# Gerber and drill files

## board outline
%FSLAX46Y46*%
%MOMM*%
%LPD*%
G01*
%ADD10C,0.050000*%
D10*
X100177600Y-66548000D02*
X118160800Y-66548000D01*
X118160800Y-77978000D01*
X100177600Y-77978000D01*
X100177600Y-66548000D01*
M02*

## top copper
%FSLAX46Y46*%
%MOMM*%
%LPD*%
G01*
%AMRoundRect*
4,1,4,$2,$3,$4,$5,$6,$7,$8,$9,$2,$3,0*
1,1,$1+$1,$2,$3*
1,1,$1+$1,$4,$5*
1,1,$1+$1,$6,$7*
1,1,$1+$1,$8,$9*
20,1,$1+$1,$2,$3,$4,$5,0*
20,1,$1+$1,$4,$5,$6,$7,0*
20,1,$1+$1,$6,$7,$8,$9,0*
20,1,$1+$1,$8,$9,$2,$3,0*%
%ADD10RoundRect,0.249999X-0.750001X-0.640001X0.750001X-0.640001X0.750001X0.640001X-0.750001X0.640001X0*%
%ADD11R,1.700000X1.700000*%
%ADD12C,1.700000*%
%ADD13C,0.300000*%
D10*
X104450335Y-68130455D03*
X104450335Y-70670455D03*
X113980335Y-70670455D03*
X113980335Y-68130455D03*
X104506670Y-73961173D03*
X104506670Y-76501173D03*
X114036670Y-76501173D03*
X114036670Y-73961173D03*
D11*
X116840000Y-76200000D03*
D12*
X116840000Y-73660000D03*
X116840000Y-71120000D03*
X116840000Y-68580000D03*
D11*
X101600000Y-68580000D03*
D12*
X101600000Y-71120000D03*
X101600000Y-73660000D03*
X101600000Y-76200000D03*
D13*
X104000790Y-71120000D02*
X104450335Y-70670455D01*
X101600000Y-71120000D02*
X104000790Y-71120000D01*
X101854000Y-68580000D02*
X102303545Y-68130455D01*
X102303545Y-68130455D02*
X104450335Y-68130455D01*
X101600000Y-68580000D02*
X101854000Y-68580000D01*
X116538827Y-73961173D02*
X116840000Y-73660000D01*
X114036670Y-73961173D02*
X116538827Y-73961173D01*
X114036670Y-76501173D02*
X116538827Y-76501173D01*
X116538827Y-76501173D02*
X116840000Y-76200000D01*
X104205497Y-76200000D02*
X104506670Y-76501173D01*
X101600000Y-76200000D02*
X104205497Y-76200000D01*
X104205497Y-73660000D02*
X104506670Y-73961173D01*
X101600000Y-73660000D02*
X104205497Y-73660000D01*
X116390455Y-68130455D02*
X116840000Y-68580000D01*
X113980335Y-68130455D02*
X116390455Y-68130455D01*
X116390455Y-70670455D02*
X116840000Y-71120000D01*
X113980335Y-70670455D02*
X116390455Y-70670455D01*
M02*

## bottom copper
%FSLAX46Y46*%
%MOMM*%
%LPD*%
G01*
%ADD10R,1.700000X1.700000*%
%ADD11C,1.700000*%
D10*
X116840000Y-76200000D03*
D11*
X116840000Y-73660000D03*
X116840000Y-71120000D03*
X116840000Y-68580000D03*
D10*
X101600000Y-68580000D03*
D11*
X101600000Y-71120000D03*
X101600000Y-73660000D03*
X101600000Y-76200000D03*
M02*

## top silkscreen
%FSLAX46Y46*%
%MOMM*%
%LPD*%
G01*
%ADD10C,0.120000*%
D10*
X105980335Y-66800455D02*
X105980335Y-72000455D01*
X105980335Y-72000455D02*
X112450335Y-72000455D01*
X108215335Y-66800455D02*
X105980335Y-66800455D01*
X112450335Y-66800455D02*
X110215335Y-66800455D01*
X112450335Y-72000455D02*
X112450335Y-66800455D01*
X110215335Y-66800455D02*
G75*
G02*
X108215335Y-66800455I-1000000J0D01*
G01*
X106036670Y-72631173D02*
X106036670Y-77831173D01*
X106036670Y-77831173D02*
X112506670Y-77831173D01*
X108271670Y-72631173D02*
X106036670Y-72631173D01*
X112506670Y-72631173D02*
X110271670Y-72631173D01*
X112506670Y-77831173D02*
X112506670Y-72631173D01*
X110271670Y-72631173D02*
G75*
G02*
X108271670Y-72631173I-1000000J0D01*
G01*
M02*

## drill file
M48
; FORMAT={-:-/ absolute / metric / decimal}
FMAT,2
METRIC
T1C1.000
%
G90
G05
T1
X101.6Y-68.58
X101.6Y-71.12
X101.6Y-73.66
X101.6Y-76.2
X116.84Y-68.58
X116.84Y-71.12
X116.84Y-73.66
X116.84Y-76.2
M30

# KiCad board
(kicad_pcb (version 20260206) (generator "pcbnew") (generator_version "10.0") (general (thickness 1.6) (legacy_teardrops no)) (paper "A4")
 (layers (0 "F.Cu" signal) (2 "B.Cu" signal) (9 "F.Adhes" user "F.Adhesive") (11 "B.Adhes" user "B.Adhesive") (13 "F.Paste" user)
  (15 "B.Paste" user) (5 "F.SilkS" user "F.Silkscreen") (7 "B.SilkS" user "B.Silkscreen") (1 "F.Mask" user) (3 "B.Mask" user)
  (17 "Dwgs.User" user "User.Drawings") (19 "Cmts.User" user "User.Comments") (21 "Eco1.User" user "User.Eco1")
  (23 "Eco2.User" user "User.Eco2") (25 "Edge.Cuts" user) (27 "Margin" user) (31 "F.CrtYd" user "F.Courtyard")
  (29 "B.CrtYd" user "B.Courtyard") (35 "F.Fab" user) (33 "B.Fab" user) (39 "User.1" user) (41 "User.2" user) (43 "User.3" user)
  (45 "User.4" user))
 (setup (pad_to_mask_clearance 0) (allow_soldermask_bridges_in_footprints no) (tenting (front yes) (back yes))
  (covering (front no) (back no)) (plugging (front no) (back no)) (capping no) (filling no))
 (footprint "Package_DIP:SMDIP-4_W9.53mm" (layer "F.Cu") (at 109.215335 69.400455)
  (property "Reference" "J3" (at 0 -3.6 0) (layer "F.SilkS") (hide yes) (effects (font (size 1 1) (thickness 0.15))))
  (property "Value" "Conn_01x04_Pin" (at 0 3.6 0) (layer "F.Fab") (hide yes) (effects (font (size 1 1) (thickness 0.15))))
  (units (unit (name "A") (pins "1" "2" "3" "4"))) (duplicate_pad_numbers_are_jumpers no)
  (fp_line (start -3.235 -2.6) (end -3.235 2.6) (stroke (width 0.12) (type solid)) (layer "F.SilkS"))
  (fp_line (start -3.235 2.6) (end 3.235 2.6) (stroke (width 0.12) (type solid)) (layer "F.SilkS"))
  (fp_line (start -1 -2.6) (end -3.235 -2.6) (stroke (width 0.12) (type solid)) (layer "F.SilkS"))
  (fp_line (start 3.235 -2.6) (end 1 -2.6) (stroke (width 0.12) (type solid)) (layer "F.SilkS"))
  (fp_line (start 3.235 2.6) (end 3.235 -2.6) (stroke (width 0.12) (type solid)) (layer "F.SilkS"))
  (fp_arc (start 1 -2.6) (mid 0 -1.6) (end -1 -2.6) (stroke (width 0.12) (type solid)) (layer "F.SilkS"))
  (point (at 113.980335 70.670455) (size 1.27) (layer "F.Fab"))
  (pad "1" smd roundrect (at -4.765 -1.27) (size 2 1.78) (layers "F.Cu" "F.Mask" "F.Paste") (roundrect_rratio 0.140449)
   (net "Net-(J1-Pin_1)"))
  (pad "2" smd roundrect (at -4.765 1.27) (size 2 1.78) (layers "F.Cu" "F.Mask" "F.Paste") (roundrect_rratio 0.140449)
   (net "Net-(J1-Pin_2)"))
  (pad "3" smd roundrect (at 4.765 1.27) (size 2 1.78) (layers "F.Cu" "F.Mask" "F.Paste") (roundrect_rratio 0.140449) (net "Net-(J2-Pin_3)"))
  (pad "4" smd roundrect (at 4.765 -1.27) (size 2 1.78) (layers "F.Cu" "F.Mask" "F.Paste") (roundrect_rratio 0.140449)
   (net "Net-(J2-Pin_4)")))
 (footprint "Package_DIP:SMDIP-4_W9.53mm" (layer "F.Cu") (at 109.27167 75.231173)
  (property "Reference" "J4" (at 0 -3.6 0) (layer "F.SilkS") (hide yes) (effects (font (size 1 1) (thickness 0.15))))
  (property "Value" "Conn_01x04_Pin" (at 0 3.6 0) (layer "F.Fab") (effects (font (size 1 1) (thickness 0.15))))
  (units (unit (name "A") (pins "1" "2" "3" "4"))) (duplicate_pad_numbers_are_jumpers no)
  (fp_line (start -3.235 -2.6) (end -3.235 2.6) (stroke (width 0.12) (type solid)) (layer "F.SilkS"))
  (fp_line (start -3.235 2.6) (end 3.235 2.6) (stroke (width 0.12) (type solid)) (layer "F.SilkS"))
  (fp_line (start -1 -2.6) (end -3.235 -2.6) (stroke (width 0.12) (type solid)) (layer "F.SilkS"))
  (fp_line (start 3.235 -2.6) (end 1 -2.6) (stroke (width 0.12) (type solid)) (layer "F.SilkS"))
  (fp_line (start 3.235 2.6) (end 3.235 -2.6) (stroke (width 0.12) (type solid)) (layer "F.SilkS"))
  (fp_arc (start 1 -2.6) (mid 0 -1.6) (end -1 -2.6) (stroke (width 0.12) (type solid)) (layer "F.SilkS"))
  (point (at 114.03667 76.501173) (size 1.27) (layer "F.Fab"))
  (pad "1" smd roundrect (at -4.765 -1.27) (size 2 1.78) (layers "F.Cu" "F.Mask" "F.Paste") (roundrect_rratio 0.140449)
   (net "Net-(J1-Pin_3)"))
  (pad "2" smd roundrect (at -4.765 1.27) (size 2 1.78) (layers "F.Cu" "F.Mask" "F.Paste") (roundrect_rratio 0.140449)
   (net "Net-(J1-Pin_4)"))
  (pad "3" smd roundrect (at 4.765 1.27) (size 2 1.78) (layers "F.Cu" "F.Mask" "F.Paste") (roundrect_rratio 0.140449) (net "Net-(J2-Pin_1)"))
  (pad "4" smd roundrect (at 4.765 -1.27) (size 2 1.78) (layers "F.Cu" "F.Mask" "F.Paste") (roundrect_rratio 0.140449)
   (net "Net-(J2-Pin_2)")))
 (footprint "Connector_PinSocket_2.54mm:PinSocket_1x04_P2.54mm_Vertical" (layer "B.Cu") (at 116.84 76.2)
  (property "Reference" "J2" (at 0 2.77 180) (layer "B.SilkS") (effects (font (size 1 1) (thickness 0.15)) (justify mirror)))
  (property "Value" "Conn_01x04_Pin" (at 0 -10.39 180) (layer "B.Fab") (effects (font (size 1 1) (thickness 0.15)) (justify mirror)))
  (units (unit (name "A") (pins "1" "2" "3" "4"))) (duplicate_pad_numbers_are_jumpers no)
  (pad "1" thru_hole rect (at 0 0) (size 1.7 1.7) (drill 1) (layers "*.Cu" "*.Mask") (remove_unused_layers no) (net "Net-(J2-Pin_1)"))
  (pad "2" thru_hole circle (at 0 -2.54) (size 1.7 1.7) (drill 1) (layers "*.Cu" "*.Mask") (remove_unused_layers no) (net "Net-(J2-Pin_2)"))
  (pad "3" thru_hole circle (at 0 -5.08) (size 1.7 1.7) (drill 1) (layers "*.Cu" "*.Mask") (remove_unused_layers no) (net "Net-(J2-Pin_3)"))
  (pad "4" thru_hole circle (at 0 -7.62) (size 1.7 1.7) (drill 1) (layers "*.Cu" "*.Mask") (remove_unused_layers no) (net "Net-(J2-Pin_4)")))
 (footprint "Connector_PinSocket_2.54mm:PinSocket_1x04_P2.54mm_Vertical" (layer "B.Cu") (at 101.6 68.58 180)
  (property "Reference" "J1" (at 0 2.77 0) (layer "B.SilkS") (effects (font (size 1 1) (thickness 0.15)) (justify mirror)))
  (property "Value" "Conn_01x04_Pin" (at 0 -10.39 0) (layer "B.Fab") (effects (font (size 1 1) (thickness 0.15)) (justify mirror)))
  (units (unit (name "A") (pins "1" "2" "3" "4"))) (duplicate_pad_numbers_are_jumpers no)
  (pad "1" thru_hole rect (at 0 0 180) (size 1.7 1.7) (drill 1) (layers "*.Cu" "*.Mask") (remove_unused_layers no) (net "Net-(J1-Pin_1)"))
  (pad "2" thru_hole circle (at 0 -2.54 180) (size 1.7 1.7) (drill 1) (layers "*.Cu" "*.Mask") (remove_unused_layers no)
   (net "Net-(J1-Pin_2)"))
  (pad "3" thru_hole circle (at 0 -5.08 180) (size 1.7 1.7) (drill 1) (layers "*.Cu" "*.Mask") (remove_unused_layers no)
   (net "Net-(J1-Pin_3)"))
  (pad "4" thru_hole circle (at 0 -7.62 180) (size 1.7 1.7) (drill 1) (layers "*.Cu" "*.Mask") (remove_unused_layers no)
   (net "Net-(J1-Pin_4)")))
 (gr_rect (start 100.1776 66.548) (end 118.1608 77.978) (stroke (width 0.05) (type default)) (fill no) (layer "Edge.Cuts"))
 (segment (start 104.00079 71.12) (end 104.450335 70.670455) (width 0.3) (layer "F.Cu") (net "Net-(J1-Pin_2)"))
 (segment (start 101.6 71.12) (end 104.00079 71.12) (width 0.3) (layer "F.Cu") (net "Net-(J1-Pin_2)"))
 (segment (start 101.854 68.58) (end 102.303545 68.130455) (width 0.3) (layer "F.Cu") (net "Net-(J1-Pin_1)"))
 (segment (start 102.303545 68.130455) (end 104.450335 68.130455) (width 0.3) (layer "F.Cu") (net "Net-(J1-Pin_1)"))
 (segment (start 101.6 68.58) (end 101.854 68.58) (width 0.3) (layer "F.Cu") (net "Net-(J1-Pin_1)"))
 (segment (start 116.538827 73.961173) (end 116.84 73.66) (width 0.3) (layer "F.Cu") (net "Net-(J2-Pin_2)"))
 (segment (start 114.03667 73.961173) (end 116.538827 73.961173) (width 0.3) (layer "F.Cu") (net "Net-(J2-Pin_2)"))
 (segment (start 114.03667 76.501173) (end 116.538827 76.501173) (width 0.3) (layer "F.Cu") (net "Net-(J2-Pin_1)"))
 (segment (start 116.538827 76.501173) (end 116.84 76.2) (width 0.3) (layer "F.Cu") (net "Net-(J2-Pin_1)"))
 (segment (start 104.205497 76.2) (end 104.50667 76.501173) (width 0.3) (layer "F.Cu") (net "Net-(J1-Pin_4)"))
 (segment (start 101.6 76.2) (end 104.205497 76.2) (width 0.3) (layer "F.Cu") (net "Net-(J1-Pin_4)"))
 (segment (start 104.205497 73.66) (end 104.50667 73.961173) (width 0.3) (layer "F.Cu") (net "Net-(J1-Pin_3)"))
 (segment (start 101.6 73.66) (end 104.205497 73.66) (width 0.3) (layer "F.Cu") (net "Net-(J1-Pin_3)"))
 (segment (start 116.390455 68.130455) (end 116.84 68.58) (width 0.3) (layer "F.Cu") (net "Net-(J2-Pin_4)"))
 (segment (start 113.980335 68.130455) (end 116.390455 68.130455) (width 0.3) (layer "F.Cu") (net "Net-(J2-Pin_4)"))
 (segment (start 116.390455 70.670455) (end 116.84 71.12) (width 0.3) (layer "F.Cu") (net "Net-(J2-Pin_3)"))
 (segment (start 113.980335 70.670455) (end 116.390455 70.670455) (width 0.3) (layer "F.Cu") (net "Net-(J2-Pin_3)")))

